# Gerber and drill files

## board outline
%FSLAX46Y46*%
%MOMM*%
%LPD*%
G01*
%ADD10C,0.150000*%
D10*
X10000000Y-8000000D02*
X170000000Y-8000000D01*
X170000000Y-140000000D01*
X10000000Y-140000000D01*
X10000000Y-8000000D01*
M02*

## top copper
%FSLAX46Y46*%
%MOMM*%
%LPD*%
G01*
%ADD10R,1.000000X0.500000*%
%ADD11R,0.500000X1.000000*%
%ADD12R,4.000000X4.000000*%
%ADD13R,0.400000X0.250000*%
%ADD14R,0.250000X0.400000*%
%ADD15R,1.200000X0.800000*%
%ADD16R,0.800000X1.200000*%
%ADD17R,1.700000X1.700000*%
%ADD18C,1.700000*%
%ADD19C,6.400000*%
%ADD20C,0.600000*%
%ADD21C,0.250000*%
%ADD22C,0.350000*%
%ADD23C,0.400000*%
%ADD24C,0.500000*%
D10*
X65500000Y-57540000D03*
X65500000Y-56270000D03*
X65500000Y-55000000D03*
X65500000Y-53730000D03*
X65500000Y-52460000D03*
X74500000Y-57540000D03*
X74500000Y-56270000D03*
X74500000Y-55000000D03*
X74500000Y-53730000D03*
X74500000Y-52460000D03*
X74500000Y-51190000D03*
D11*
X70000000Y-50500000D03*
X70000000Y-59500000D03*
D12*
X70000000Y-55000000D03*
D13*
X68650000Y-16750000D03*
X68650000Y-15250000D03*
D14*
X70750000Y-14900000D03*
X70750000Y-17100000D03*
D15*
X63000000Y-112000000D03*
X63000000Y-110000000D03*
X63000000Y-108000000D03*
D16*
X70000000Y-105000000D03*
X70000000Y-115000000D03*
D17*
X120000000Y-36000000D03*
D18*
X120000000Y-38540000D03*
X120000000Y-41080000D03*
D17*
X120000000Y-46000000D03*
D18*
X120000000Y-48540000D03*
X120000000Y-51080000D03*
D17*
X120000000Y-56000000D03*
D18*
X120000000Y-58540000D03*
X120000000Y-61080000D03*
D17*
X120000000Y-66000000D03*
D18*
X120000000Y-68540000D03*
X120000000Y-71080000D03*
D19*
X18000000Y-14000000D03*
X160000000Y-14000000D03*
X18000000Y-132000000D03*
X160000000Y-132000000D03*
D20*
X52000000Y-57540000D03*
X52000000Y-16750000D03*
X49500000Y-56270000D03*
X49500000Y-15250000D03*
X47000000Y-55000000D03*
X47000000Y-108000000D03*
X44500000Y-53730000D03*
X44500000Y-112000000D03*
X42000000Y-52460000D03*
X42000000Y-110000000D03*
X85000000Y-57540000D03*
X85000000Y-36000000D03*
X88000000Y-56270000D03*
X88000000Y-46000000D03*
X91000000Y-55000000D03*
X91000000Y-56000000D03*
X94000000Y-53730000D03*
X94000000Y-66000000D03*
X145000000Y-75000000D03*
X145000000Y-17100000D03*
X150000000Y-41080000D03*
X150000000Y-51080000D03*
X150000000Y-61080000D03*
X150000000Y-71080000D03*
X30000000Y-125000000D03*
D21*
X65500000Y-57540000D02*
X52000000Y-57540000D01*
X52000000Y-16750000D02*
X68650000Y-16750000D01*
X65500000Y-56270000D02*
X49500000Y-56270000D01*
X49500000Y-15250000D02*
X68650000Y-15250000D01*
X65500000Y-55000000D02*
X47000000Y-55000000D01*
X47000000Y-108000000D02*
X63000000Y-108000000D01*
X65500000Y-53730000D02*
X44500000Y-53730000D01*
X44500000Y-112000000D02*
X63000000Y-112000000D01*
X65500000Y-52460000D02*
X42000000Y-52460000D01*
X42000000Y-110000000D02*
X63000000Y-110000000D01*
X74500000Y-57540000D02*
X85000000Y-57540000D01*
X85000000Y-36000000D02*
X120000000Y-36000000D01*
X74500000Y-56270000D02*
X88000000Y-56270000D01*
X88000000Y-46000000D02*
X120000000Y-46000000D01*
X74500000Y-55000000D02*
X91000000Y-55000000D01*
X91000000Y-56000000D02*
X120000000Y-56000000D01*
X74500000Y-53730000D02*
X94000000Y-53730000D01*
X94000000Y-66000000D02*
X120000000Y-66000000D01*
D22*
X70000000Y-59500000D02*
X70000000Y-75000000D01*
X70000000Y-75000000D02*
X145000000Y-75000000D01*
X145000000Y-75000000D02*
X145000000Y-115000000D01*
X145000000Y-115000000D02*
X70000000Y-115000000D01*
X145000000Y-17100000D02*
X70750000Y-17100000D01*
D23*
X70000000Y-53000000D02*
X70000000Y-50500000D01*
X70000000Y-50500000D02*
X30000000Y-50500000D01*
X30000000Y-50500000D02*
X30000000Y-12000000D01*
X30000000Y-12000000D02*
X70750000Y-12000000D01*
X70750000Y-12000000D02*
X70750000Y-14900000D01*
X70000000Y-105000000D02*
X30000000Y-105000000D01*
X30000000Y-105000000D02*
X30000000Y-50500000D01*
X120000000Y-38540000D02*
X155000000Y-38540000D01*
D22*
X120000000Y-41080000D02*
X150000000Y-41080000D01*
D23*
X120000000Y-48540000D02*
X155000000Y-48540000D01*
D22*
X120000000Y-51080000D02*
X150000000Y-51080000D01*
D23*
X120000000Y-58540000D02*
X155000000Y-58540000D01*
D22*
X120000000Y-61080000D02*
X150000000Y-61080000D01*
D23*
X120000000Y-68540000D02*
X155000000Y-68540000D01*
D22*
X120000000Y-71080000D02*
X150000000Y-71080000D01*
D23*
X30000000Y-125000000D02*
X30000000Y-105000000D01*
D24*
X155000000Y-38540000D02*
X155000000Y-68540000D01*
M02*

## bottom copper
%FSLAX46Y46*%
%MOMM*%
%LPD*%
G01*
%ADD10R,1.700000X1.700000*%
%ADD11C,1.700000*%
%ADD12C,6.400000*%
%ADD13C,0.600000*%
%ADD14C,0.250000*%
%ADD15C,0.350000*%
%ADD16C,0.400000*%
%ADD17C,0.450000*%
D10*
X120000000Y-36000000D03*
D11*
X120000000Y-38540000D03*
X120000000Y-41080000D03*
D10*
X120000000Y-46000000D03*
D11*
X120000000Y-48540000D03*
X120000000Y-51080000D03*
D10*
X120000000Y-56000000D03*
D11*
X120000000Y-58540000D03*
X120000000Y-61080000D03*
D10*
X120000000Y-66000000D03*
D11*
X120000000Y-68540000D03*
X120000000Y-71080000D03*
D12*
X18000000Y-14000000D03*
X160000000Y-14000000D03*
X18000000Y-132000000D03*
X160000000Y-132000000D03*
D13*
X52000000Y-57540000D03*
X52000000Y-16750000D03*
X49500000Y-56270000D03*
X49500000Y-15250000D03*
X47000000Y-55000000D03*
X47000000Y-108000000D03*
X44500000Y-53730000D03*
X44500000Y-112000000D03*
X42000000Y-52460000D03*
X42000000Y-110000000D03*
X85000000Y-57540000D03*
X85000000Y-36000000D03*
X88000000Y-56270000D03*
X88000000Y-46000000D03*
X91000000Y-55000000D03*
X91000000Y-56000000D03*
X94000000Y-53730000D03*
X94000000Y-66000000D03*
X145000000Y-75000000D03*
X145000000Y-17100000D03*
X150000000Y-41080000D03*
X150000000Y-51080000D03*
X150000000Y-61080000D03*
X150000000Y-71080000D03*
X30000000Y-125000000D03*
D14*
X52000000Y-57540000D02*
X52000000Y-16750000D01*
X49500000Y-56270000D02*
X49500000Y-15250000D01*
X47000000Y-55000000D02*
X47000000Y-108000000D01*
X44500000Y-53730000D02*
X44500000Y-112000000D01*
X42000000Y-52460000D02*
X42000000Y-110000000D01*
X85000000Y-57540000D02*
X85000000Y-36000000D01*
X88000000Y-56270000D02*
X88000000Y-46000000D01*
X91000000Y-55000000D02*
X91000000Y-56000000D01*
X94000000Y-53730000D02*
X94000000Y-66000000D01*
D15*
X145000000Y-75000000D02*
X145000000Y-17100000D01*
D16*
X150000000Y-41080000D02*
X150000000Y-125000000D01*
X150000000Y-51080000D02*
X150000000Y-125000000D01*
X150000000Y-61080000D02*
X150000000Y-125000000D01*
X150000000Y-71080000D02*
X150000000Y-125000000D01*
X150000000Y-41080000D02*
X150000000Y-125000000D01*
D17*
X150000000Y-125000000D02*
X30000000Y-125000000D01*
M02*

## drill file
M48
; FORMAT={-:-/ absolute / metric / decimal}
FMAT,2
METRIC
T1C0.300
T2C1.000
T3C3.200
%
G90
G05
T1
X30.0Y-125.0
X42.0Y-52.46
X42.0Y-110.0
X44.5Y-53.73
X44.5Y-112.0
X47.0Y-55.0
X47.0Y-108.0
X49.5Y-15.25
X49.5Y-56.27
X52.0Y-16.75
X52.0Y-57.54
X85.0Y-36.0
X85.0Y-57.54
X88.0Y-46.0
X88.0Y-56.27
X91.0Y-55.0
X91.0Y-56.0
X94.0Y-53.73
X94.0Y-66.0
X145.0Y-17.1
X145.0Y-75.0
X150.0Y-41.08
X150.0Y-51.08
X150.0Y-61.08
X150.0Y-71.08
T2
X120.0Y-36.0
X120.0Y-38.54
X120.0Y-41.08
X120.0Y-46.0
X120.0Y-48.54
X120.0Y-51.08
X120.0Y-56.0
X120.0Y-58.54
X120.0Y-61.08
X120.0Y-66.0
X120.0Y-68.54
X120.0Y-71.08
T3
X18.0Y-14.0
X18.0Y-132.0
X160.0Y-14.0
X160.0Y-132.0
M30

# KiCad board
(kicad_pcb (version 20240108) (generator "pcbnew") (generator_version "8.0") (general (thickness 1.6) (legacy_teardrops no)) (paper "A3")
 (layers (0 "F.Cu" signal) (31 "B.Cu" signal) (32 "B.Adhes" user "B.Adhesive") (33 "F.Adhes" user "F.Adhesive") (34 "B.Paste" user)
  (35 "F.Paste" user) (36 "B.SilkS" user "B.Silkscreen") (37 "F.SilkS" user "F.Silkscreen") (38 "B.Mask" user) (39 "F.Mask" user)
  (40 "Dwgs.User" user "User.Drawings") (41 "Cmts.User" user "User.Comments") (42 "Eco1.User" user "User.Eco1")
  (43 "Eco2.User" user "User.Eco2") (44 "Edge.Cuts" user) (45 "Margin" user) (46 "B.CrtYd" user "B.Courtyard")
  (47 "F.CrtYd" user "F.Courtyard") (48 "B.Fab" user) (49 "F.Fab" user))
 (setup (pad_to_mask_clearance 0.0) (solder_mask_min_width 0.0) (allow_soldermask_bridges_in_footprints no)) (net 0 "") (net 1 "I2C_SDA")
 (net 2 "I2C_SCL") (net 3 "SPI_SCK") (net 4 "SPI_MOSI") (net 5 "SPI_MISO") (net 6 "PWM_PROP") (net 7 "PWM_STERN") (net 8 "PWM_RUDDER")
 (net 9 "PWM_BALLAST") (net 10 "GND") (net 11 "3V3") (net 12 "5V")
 (gr_rect (start 10 8) (end 170 140) (stroke (width 0.15) (type solid)) (fill none) (layer "Edge.Cuts"))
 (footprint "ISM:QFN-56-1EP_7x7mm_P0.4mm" (layer "F.Cu") (at 70 55)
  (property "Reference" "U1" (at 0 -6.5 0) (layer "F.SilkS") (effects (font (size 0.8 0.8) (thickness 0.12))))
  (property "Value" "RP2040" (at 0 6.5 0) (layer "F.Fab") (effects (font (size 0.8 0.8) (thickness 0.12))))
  (pad "1" smd rect (at -4.5 2.54) (size 1.0 0.5) (layers "F.Cu" "F.Paste" "F.Mask") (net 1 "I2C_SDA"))
  (pad "2" smd rect (at -4.5 1.27) (size 1.0 0.5) (layers "F.Cu" "F.Paste" "F.Mask") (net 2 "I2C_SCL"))
  (pad "3" smd rect (at -4.5 0) (size 1.0 0.5) (layers "F.Cu" "F.Paste" "F.Mask") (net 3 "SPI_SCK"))
  (pad "4" smd rect (at -4.5 -1.27) (size 1.0 0.5) (layers "F.Cu" "F.Paste" "F.Mask") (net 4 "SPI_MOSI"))
  (pad "5" smd rect (at -4.5 -2.54) (size 1.0 0.5) (layers "F.Cu" "F.Paste" "F.Mask") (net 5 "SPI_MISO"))
  (pad "6" smd rect (at 4.5 2.54) (size 1.0 0.5) (layers "F.Cu" "F.Paste" "F.Mask") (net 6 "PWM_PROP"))
  (pad "7" smd rect (at 4.5 1.27) (size 1.0 0.5) (layers "F.Cu" "F.Paste" "F.Mask") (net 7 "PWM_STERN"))
  (pad "8" smd rect (at 4.5 0) (size 1.0 0.5) (layers "F.Cu" "F.Paste" "F.Mask") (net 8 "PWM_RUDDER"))
  (pad "9" smd rect (at 4.5 -1.27) (size 1.0 0.5) (layers "F.Cu" "F.Paste" "F.Mask") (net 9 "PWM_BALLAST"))
  (pad "12" smd rect (at 4.5 -2.54) (size 1.0 0.5) (layers "F.Cu" "F.Paste" "F.Mask"))
  (pad "13" smd rect (at 4.5 -3.81) (size 1.0 0.5) (layers "F.Cu" "F.Paste" "F.Mask"))
  (pad "10" smd rect (at 0 -4.5) (size 0.5 1.0) (layers "F.Cu" "F.Paste" "F.Mask") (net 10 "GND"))
  (pad "11" smd rect (at 0 4.5) (size 0.5 1.0) (layers "F.Cu" "F.Paste" "F.Mask") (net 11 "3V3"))
  (pad "EP" smd rect (at 0 0) (size 4 4) (layers "F.Cu" "F.Paste" "F.Mask") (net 10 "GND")))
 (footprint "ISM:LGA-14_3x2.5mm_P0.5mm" (layer "F.Cu") (at 70 16)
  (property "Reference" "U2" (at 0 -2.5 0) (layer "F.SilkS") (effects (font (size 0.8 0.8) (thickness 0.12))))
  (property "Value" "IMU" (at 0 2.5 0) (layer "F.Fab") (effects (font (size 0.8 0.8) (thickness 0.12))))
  (pad "1" smd rect (at -1.35 0.75) (size 0.4 0.25) (layers "F.Cu" "F.Paste" "F.Mask") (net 1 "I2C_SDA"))
  (pad "2" smd rect (at -1.35 -0.75) (size 0.4 0.25) (layers "F.Cu" "F.Paste" "F.Mask") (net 2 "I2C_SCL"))
  (pad "3" smd rect (at 0.75 -1.1) (size 0.25 0.4) (layers "F.Cu" "F.Paste" "F.Mask") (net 10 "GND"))
  (pad "4" smd rect (at 0.75 1.1) (size 0.25 0.4) (layers "F.Cu" "F.Paste" "F.Mask") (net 11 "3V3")))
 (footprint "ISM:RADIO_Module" (layer "F.Cu") (at 70 110)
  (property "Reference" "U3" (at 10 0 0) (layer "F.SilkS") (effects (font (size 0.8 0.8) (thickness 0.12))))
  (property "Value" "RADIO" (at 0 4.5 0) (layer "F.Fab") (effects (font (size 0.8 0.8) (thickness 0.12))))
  (pad "1" smd rect (at -7 2) (size 1.2 0.8) (layers "F.Cu" "F.Paste" "F.Mask") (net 4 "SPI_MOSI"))
  (pad "2" smd rect (at -7 0) (size 1.2 0.8) (layers "F.Cu" "F.Paste" "F.Mask") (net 5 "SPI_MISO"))
  (pad "3" smd rect (at -7 -2) (size 1.2 0.8) (layers "F.Cu" "F.Paste" "F.Mask") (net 3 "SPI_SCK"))
  (pad "4" smd rect (at 0 -5) (size 0.8 1.2) (layers "F.Cu" "F.Paste" "F.Mask") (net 10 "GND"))
  (pad "5" smd rect (at 0 5) (size 0.8 1.2) (layers "F.Cu" "F.Paste" "F.Mask") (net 11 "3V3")))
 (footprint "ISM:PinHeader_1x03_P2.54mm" (layer "F.Cu") (at 120 36)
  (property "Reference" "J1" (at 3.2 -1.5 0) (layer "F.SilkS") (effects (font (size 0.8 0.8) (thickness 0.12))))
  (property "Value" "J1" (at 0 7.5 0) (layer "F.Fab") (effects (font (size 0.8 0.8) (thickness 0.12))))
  (pad "1" thru_hole rect (at 0 0) (size 1.7 1.7) (drill 1.0) (layers "*.Cu" "*.Mask") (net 6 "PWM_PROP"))
  (pad "2" thru_hole circle (at 0 2.54) (size 1.7 1.7) (drill 1.0) (layers "*.Cu" "*.Mask") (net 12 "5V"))
  (pad "3" thru_hole circle (at 0 5.08) (size 1.7 1.7) (drill 1.0) (layers "*.Cu" "*.Mask") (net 10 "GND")))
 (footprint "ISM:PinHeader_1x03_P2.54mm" (layer "F.Cu") (at 120 46)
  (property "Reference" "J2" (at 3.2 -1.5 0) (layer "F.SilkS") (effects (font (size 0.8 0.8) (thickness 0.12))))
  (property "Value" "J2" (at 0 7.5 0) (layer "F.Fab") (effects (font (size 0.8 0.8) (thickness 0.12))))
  (pad "1" thru_hole rect (at 0 0) (size 1.7 1.7) (drill 1.0) (layers "*.Cu" "*.Mask") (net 7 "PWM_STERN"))
  (pad "2" thru_hole circle (at 0 2.54) (size 1.7 1.7) (drill 1.0) (layers "*.Cu" "*.Mask") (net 12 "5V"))
  (pad "3" thru_hole circle (at 0 5.08) (size 1.7 1.7) (drill 1.0) (layers "*.Cu" "*.Mask") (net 10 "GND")))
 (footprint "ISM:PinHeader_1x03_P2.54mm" (layer "F.Cu") (at 120 56)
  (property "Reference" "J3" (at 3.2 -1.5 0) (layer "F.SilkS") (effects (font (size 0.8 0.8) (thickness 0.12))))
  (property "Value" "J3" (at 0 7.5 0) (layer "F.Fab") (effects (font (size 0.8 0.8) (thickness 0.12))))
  (pad "1" thru_hole rect (at 0 0) (size 1.7 1.7) (drill 1.0) (layers "*.Cu" "*.Mask") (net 8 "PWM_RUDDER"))
  (pad "2" thru_hole circle (at 0 2.54) (size 1.7 1.7) (drill 1.0) (layers "*.Cu" "*.Mask") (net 12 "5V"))
  (pad "3" thru_hole circle (at 0 5.08) (size 1.7 1.7) (drill 1.0) (layers "*.Cu" "*.Mask") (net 10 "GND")))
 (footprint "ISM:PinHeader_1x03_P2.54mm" (layer "F.Cu") (at 120 66)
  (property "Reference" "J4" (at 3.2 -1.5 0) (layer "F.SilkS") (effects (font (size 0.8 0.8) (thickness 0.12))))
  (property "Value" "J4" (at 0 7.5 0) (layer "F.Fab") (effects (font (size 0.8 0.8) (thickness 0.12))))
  (pad "1" thru_hole rect (at 0 0) (size 1.7 1.7) (drill 1.0) (layers "*.Cu" "*.Mask") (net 9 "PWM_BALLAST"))
  (pad "2" thru_hole circle (at 0 2.54) (size 1.7 1.7) (drill 1.0) (layers "*.Cu" "*.Mask") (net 12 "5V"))
  (pad "3" thru_hole circle (at 0 5.08) (size 1.7 1.7) (drill 1.0) (layers "*.Cu" "*.Mask") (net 10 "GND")))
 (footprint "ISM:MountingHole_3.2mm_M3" (layer "F.Cu") (at 18 14)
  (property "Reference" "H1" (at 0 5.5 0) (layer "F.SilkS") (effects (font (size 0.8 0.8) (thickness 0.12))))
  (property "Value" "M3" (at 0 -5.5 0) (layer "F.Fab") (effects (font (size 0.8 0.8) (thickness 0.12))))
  (pad "" thru_hole circle (at 0 0) (size 6.4 6.4) (drill 3.2) (layers "*.Cu" "*.Mask")))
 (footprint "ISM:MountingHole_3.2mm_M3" (layer "F.Cu") (at 160 14)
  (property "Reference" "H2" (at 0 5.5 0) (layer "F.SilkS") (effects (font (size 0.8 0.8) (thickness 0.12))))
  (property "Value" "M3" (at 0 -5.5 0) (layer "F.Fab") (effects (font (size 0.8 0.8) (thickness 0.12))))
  (pad "" thru_hole circle (at 0 0) (size 6.4 6.4) (drill 3.2) (layers "*.Cu" "*.Mask")))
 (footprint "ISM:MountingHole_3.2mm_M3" (layer "F.Cu") (at 18 132)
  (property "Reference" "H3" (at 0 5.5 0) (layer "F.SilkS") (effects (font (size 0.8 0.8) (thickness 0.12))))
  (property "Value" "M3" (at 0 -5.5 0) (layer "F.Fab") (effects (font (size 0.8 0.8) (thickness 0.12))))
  (pad "" thru_hole circle (at 0 0) (size 6.4 6.4) (drill 3.2) (layers "*.Cu" "*.Mask")))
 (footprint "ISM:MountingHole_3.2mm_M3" (layer "F.Cu") (at 160 132)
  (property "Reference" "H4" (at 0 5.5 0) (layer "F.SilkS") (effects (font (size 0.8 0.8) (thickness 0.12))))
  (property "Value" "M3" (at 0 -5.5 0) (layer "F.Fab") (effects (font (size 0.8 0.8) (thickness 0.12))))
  (pad "" thru_hole circle (at 0 0) (size 6.4 6.4) (drill 3.2) (layers "*.Cu" "*.Mask")))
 (segment (start 65.5 57.54) (end 52.0 57.54) (width 0.25) (layer "F.Cu") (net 1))
 (segment (start 52.0 57.54) (end 52.0 16.75) (width 0.25) (layer "B.Cu") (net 1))
 (segment (start 52.0 16.75) (end 68.65 16.75) (width 0.25) (layer "F.Cu") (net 1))
 (segment (start 65.5 56.27) (end 49.5 56.27) (width 0.25) (layer "F.Cu") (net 2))
 (segment (start 49.5 56.27) (end 49.5 15.25) (width 0.25) (layer "B.Cu") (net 2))
 (segment (start 49.5 15.25) (end 68.65 15.25) (width 0.25) (layer "F.Cu") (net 2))
 (segment (start 65.5 55) (end 47.0 55) (width 0.25) (layer "F.Cu") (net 3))
 (segment (start 47.0 55) (end 47.0 108) (width 0.25) (layer "B.Cu") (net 3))
 (segment (start 47.0 108) (end 63 108) (width 0.25) (layer "F.Cu") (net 3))
 (segment (start 65.5 53.73) (end 44.5 53.73) (width 0.25) (layer "F.Cu") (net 4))
 (segment (start 44.5 53.73) (end 44.5 112) (width 0.25) (layer "B.Cu") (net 4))
 (segment (start 44.5 112) (end 63 112) (width 0.25) (layer "F.Cu") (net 4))
 (segment (start 65.5 52.46) (end 42.0 52.46) (width 0.25) (layer "F.Cu") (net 5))
 (segment (start 42.0 52.46) (end 42.0 110) (width 0.25) (layer "B.Cu") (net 5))
 (segment (start 42.0 110) (end 63 110) (width 0.25) (layer "F.Cu") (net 5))
 (segment (start 74.5 57.54) (end 85 57.54) (width 0.25) (layer "F.Cu") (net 6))
 (segment (start 85 57.54) (end 85 36) (width 0.25) (layer "B.Cu") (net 6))
 (segment (start 85 36) (end 120 36) (width 0.25) (layer "F.Cu") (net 6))
 (segment (start 74.5 56.27) (end 88 56.27) (width 0.25) (layer "F.Cu") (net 7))
 (segment (start 88 56.27) (end 88 46) (width 0.25) (layer "B.Cu") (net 7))
 (segment (start 88 46) (end 120 46) (width 0.25) (layer "F.Cu") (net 7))
 (segment (start 74.5 55) (end 91 55) (width 0.25) (layer "F.Cu") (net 8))
 (segment (start 91 55) (end 91 56) (width 0.25) (layer "B.Cu") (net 8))
 (segment (start 91 56) (end 120 56) (width 0.25) (layer "F.Cu") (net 8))
 (segment (start 74.5 53.73) (end 94 53.73) (width 0.25) (layer "F.Cu") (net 9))
 (segment (start 94 53.73) (end 94 66) (width 0.25) (layer "B.Cu") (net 9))
 (segment (start 94 66) (end 120 66) (width 0.25) (layer "F.Cu") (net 9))
 (segment (start 70 59.5) (end 70 75) (width 0.35) (layer "F.Cu") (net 11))
 (segment (start 70 75) (end 145 75) (width 0.35) (layer "F.Cu") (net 11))
 (segment (start 145 75) (end 145 115) (width 0.35) (layer "F.Cu") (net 11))
 (segment (start 145 115) (end 70 115) (width 0.35) (layer "F.Cu") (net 11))
 (segment (start 145 75) (end 145 17.1) (width 0.35) (layer "B.Cu") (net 11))
 (segment (start 145 17.1) (end 70.75 17.1) (width 0.35) (layer "F.Cu") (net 11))
 (segment (start 70 53) (end 70 50.5) (width 0.4) (layer "F.Cu") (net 10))
 (segment (start 70 50.5) (end 30 50.5) (width 0.4) (layer "F.Cu") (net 10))
 (segment (start 30 50.5) (end 30 12) (width 0.4) (layer "F.Cu") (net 10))
 (segment (start 30 12) (end 70.75 12) (width 0.4) (layer "F.Cu") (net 10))
 (segment (start 70.75 12) (end 70.75 14.9) (width 0.4) (layer "F.Cu") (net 10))
 (segment (start 70 105) (end 30 105) (width 0.4) (layer "F.Cu") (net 10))
 (segment (start 30 105) (end 30 50.5) (width 0.4) (layer "F.Cu") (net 10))
 (segment (start 120 38.54) (end 155 38.54) (width 0.4) (layer "F.Cu") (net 12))
 (segment (start 120 41.08) (end 150 41.08) (width 0.35) (layer "F.Cu") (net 10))
 (segment (start 150 41.08) (end 150 125) (width 0.4) (layer "B.Cu") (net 10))
 (segment (start 120 48.54) (end 155 48.54) (width 0.4) (layer "F.Cu") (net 12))
 (segment (start 120 51.08) (end 150 51.08) (width 0.35) (layer "F.Cu") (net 10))
 (segment (start 150 51.08) (end 150 125) (width 0.4) (layer "B.Cu") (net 10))
 (segment (start 120 58.54) (end 155 58.54) (width 0.4) (layer "F.Cu") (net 12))
 (segment (start 120 61.08) (end 150 61.08) (width 0.35) (layer "F.Cu") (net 10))
 (segment (start 150 61.08) (end 150 125) (width 0.4) (layer "B.Cu") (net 10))
 (segment (start 120 68.54) (end 155 68.54) (width 0.4) (layer "F.Cu") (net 12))
 (segment (start 120 71.08) (end 150 71.08) (width 0.35) (layer "F.Cu") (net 10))
 (segment (start 150 71.08) (end 150 125) (width 0.4) (layer "B.Cu") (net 10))
 (segment (start 150 41.08) (end 150 125) (width 0.4) (layer "B.Cu") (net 10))
 (segment (start 150 125) (end 30 125) (width 0.45) (layer "B.Cu") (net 10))
 (segment (start 30 125) (end 30 105) (width 0.4) (layer "F.Cu") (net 10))
 (segment (start 155 38.54) (end 155 68.54) (width 0.5) (layer "F.Cu") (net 12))
 (via (at 52.0 57.54) (size 0.6) (drill 0.3) (layers "F.Cu" "B.Cu") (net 1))
 (via (at 52.0 16.75) (size 0.6) (drill 0.3) (layers "F.Cu" "B.Cu") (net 1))
 (via (at 49.5 56.27) (size 0.6) (drill 0.3) (layers "F.Cu" "B.Cu") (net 2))
 (via (at 49.5 15.25) (size 0.6) (drill 0.3) (layers "F.Cu" "B.Cu") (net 2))
 (via (at 47.0 55) (size 0.6) (drill 0.3) (layers "F.Cu" "B.Cu") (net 3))
 (via (at 47.0 108) (size 0.6) (drill 0.3) (layers "F.Cu" "B.Cu") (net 3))
 (via (at 44.5 53.73) (size 0.6) (drill 0.3) (layers "F.Cu" "B.Cu") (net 4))
 (via (at 44.5 112) (size 0.6) (drill 0.3) (layers "F.Cu" "B.Cu") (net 4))
 (via (at 42.0 52.46) (size 0.6) (drill 0.3) (layers "F.Cu" "B.Cu") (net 5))
 (via (at 42.0 110) (size 0.6) (drill 0.3) (layers "F.Cu" "B.Cu") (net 5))
 (via (at 85 57.54) (size 0.6) (drill 0.3) (layers "F.Cu" "B.Cu") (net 6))
 (via (at 85 36) (size 0.6) (drill 0.3) (layers "F.Cu" "B.Cu") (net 6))
 (via (at 88 56.27) (size 0.6) (drill 0.3) (layers "F.Cu" "B.Cu") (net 7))
 (via (at 88 46) (size 0.6) (drill 0.3) (layers "F.Cu" "B.Cu") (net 7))
 (via (at 91 55) (size 0.6) (drill 0.3) (layers "F.Cu" "B.Cu") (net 8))
 (via (at 91 56) (size 0.6) (drill 0.3) (layers "F.Cu" "B.Cu") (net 8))
 (via (at 94 53.73) (size 0.6) (drill 0.3) (layers "F.Cu" "B.Cu") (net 9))
 (via (at 94 66) (size 0.6) (drill 0.3) (layers "F.Cu" "B.Cu") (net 9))
 (via (at 145 75) (size 0.6) (drill 0.3) (layers "F.Cu" "B.Cu") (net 11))
 (via (at 145 17.1) (size 0.6) (drill 0.3) (layers "F.Cu" "B.Cu") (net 11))
 (via (at 150 41.08) (size 0.6) (drill 0.3) (layers "F.Cu" "B.Cu") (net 10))
 (via (at 150 51.08) (size 0.6) (drill 0.3) (layers "F.Cu" "B.Cu") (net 10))
 (via (at 150 61.08) (size 0.6) (drill 0.3) (layers "F.Cu" "B.Cu") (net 10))
 (via (at 150 71.08) (size 0.6) (drill 0.3) (layers "F.Cu" "B.Cu") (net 10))
 (via (at 30 125) (size 0.6) (drill 0.3) (layers "F.Cu" "B.Cu") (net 10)))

